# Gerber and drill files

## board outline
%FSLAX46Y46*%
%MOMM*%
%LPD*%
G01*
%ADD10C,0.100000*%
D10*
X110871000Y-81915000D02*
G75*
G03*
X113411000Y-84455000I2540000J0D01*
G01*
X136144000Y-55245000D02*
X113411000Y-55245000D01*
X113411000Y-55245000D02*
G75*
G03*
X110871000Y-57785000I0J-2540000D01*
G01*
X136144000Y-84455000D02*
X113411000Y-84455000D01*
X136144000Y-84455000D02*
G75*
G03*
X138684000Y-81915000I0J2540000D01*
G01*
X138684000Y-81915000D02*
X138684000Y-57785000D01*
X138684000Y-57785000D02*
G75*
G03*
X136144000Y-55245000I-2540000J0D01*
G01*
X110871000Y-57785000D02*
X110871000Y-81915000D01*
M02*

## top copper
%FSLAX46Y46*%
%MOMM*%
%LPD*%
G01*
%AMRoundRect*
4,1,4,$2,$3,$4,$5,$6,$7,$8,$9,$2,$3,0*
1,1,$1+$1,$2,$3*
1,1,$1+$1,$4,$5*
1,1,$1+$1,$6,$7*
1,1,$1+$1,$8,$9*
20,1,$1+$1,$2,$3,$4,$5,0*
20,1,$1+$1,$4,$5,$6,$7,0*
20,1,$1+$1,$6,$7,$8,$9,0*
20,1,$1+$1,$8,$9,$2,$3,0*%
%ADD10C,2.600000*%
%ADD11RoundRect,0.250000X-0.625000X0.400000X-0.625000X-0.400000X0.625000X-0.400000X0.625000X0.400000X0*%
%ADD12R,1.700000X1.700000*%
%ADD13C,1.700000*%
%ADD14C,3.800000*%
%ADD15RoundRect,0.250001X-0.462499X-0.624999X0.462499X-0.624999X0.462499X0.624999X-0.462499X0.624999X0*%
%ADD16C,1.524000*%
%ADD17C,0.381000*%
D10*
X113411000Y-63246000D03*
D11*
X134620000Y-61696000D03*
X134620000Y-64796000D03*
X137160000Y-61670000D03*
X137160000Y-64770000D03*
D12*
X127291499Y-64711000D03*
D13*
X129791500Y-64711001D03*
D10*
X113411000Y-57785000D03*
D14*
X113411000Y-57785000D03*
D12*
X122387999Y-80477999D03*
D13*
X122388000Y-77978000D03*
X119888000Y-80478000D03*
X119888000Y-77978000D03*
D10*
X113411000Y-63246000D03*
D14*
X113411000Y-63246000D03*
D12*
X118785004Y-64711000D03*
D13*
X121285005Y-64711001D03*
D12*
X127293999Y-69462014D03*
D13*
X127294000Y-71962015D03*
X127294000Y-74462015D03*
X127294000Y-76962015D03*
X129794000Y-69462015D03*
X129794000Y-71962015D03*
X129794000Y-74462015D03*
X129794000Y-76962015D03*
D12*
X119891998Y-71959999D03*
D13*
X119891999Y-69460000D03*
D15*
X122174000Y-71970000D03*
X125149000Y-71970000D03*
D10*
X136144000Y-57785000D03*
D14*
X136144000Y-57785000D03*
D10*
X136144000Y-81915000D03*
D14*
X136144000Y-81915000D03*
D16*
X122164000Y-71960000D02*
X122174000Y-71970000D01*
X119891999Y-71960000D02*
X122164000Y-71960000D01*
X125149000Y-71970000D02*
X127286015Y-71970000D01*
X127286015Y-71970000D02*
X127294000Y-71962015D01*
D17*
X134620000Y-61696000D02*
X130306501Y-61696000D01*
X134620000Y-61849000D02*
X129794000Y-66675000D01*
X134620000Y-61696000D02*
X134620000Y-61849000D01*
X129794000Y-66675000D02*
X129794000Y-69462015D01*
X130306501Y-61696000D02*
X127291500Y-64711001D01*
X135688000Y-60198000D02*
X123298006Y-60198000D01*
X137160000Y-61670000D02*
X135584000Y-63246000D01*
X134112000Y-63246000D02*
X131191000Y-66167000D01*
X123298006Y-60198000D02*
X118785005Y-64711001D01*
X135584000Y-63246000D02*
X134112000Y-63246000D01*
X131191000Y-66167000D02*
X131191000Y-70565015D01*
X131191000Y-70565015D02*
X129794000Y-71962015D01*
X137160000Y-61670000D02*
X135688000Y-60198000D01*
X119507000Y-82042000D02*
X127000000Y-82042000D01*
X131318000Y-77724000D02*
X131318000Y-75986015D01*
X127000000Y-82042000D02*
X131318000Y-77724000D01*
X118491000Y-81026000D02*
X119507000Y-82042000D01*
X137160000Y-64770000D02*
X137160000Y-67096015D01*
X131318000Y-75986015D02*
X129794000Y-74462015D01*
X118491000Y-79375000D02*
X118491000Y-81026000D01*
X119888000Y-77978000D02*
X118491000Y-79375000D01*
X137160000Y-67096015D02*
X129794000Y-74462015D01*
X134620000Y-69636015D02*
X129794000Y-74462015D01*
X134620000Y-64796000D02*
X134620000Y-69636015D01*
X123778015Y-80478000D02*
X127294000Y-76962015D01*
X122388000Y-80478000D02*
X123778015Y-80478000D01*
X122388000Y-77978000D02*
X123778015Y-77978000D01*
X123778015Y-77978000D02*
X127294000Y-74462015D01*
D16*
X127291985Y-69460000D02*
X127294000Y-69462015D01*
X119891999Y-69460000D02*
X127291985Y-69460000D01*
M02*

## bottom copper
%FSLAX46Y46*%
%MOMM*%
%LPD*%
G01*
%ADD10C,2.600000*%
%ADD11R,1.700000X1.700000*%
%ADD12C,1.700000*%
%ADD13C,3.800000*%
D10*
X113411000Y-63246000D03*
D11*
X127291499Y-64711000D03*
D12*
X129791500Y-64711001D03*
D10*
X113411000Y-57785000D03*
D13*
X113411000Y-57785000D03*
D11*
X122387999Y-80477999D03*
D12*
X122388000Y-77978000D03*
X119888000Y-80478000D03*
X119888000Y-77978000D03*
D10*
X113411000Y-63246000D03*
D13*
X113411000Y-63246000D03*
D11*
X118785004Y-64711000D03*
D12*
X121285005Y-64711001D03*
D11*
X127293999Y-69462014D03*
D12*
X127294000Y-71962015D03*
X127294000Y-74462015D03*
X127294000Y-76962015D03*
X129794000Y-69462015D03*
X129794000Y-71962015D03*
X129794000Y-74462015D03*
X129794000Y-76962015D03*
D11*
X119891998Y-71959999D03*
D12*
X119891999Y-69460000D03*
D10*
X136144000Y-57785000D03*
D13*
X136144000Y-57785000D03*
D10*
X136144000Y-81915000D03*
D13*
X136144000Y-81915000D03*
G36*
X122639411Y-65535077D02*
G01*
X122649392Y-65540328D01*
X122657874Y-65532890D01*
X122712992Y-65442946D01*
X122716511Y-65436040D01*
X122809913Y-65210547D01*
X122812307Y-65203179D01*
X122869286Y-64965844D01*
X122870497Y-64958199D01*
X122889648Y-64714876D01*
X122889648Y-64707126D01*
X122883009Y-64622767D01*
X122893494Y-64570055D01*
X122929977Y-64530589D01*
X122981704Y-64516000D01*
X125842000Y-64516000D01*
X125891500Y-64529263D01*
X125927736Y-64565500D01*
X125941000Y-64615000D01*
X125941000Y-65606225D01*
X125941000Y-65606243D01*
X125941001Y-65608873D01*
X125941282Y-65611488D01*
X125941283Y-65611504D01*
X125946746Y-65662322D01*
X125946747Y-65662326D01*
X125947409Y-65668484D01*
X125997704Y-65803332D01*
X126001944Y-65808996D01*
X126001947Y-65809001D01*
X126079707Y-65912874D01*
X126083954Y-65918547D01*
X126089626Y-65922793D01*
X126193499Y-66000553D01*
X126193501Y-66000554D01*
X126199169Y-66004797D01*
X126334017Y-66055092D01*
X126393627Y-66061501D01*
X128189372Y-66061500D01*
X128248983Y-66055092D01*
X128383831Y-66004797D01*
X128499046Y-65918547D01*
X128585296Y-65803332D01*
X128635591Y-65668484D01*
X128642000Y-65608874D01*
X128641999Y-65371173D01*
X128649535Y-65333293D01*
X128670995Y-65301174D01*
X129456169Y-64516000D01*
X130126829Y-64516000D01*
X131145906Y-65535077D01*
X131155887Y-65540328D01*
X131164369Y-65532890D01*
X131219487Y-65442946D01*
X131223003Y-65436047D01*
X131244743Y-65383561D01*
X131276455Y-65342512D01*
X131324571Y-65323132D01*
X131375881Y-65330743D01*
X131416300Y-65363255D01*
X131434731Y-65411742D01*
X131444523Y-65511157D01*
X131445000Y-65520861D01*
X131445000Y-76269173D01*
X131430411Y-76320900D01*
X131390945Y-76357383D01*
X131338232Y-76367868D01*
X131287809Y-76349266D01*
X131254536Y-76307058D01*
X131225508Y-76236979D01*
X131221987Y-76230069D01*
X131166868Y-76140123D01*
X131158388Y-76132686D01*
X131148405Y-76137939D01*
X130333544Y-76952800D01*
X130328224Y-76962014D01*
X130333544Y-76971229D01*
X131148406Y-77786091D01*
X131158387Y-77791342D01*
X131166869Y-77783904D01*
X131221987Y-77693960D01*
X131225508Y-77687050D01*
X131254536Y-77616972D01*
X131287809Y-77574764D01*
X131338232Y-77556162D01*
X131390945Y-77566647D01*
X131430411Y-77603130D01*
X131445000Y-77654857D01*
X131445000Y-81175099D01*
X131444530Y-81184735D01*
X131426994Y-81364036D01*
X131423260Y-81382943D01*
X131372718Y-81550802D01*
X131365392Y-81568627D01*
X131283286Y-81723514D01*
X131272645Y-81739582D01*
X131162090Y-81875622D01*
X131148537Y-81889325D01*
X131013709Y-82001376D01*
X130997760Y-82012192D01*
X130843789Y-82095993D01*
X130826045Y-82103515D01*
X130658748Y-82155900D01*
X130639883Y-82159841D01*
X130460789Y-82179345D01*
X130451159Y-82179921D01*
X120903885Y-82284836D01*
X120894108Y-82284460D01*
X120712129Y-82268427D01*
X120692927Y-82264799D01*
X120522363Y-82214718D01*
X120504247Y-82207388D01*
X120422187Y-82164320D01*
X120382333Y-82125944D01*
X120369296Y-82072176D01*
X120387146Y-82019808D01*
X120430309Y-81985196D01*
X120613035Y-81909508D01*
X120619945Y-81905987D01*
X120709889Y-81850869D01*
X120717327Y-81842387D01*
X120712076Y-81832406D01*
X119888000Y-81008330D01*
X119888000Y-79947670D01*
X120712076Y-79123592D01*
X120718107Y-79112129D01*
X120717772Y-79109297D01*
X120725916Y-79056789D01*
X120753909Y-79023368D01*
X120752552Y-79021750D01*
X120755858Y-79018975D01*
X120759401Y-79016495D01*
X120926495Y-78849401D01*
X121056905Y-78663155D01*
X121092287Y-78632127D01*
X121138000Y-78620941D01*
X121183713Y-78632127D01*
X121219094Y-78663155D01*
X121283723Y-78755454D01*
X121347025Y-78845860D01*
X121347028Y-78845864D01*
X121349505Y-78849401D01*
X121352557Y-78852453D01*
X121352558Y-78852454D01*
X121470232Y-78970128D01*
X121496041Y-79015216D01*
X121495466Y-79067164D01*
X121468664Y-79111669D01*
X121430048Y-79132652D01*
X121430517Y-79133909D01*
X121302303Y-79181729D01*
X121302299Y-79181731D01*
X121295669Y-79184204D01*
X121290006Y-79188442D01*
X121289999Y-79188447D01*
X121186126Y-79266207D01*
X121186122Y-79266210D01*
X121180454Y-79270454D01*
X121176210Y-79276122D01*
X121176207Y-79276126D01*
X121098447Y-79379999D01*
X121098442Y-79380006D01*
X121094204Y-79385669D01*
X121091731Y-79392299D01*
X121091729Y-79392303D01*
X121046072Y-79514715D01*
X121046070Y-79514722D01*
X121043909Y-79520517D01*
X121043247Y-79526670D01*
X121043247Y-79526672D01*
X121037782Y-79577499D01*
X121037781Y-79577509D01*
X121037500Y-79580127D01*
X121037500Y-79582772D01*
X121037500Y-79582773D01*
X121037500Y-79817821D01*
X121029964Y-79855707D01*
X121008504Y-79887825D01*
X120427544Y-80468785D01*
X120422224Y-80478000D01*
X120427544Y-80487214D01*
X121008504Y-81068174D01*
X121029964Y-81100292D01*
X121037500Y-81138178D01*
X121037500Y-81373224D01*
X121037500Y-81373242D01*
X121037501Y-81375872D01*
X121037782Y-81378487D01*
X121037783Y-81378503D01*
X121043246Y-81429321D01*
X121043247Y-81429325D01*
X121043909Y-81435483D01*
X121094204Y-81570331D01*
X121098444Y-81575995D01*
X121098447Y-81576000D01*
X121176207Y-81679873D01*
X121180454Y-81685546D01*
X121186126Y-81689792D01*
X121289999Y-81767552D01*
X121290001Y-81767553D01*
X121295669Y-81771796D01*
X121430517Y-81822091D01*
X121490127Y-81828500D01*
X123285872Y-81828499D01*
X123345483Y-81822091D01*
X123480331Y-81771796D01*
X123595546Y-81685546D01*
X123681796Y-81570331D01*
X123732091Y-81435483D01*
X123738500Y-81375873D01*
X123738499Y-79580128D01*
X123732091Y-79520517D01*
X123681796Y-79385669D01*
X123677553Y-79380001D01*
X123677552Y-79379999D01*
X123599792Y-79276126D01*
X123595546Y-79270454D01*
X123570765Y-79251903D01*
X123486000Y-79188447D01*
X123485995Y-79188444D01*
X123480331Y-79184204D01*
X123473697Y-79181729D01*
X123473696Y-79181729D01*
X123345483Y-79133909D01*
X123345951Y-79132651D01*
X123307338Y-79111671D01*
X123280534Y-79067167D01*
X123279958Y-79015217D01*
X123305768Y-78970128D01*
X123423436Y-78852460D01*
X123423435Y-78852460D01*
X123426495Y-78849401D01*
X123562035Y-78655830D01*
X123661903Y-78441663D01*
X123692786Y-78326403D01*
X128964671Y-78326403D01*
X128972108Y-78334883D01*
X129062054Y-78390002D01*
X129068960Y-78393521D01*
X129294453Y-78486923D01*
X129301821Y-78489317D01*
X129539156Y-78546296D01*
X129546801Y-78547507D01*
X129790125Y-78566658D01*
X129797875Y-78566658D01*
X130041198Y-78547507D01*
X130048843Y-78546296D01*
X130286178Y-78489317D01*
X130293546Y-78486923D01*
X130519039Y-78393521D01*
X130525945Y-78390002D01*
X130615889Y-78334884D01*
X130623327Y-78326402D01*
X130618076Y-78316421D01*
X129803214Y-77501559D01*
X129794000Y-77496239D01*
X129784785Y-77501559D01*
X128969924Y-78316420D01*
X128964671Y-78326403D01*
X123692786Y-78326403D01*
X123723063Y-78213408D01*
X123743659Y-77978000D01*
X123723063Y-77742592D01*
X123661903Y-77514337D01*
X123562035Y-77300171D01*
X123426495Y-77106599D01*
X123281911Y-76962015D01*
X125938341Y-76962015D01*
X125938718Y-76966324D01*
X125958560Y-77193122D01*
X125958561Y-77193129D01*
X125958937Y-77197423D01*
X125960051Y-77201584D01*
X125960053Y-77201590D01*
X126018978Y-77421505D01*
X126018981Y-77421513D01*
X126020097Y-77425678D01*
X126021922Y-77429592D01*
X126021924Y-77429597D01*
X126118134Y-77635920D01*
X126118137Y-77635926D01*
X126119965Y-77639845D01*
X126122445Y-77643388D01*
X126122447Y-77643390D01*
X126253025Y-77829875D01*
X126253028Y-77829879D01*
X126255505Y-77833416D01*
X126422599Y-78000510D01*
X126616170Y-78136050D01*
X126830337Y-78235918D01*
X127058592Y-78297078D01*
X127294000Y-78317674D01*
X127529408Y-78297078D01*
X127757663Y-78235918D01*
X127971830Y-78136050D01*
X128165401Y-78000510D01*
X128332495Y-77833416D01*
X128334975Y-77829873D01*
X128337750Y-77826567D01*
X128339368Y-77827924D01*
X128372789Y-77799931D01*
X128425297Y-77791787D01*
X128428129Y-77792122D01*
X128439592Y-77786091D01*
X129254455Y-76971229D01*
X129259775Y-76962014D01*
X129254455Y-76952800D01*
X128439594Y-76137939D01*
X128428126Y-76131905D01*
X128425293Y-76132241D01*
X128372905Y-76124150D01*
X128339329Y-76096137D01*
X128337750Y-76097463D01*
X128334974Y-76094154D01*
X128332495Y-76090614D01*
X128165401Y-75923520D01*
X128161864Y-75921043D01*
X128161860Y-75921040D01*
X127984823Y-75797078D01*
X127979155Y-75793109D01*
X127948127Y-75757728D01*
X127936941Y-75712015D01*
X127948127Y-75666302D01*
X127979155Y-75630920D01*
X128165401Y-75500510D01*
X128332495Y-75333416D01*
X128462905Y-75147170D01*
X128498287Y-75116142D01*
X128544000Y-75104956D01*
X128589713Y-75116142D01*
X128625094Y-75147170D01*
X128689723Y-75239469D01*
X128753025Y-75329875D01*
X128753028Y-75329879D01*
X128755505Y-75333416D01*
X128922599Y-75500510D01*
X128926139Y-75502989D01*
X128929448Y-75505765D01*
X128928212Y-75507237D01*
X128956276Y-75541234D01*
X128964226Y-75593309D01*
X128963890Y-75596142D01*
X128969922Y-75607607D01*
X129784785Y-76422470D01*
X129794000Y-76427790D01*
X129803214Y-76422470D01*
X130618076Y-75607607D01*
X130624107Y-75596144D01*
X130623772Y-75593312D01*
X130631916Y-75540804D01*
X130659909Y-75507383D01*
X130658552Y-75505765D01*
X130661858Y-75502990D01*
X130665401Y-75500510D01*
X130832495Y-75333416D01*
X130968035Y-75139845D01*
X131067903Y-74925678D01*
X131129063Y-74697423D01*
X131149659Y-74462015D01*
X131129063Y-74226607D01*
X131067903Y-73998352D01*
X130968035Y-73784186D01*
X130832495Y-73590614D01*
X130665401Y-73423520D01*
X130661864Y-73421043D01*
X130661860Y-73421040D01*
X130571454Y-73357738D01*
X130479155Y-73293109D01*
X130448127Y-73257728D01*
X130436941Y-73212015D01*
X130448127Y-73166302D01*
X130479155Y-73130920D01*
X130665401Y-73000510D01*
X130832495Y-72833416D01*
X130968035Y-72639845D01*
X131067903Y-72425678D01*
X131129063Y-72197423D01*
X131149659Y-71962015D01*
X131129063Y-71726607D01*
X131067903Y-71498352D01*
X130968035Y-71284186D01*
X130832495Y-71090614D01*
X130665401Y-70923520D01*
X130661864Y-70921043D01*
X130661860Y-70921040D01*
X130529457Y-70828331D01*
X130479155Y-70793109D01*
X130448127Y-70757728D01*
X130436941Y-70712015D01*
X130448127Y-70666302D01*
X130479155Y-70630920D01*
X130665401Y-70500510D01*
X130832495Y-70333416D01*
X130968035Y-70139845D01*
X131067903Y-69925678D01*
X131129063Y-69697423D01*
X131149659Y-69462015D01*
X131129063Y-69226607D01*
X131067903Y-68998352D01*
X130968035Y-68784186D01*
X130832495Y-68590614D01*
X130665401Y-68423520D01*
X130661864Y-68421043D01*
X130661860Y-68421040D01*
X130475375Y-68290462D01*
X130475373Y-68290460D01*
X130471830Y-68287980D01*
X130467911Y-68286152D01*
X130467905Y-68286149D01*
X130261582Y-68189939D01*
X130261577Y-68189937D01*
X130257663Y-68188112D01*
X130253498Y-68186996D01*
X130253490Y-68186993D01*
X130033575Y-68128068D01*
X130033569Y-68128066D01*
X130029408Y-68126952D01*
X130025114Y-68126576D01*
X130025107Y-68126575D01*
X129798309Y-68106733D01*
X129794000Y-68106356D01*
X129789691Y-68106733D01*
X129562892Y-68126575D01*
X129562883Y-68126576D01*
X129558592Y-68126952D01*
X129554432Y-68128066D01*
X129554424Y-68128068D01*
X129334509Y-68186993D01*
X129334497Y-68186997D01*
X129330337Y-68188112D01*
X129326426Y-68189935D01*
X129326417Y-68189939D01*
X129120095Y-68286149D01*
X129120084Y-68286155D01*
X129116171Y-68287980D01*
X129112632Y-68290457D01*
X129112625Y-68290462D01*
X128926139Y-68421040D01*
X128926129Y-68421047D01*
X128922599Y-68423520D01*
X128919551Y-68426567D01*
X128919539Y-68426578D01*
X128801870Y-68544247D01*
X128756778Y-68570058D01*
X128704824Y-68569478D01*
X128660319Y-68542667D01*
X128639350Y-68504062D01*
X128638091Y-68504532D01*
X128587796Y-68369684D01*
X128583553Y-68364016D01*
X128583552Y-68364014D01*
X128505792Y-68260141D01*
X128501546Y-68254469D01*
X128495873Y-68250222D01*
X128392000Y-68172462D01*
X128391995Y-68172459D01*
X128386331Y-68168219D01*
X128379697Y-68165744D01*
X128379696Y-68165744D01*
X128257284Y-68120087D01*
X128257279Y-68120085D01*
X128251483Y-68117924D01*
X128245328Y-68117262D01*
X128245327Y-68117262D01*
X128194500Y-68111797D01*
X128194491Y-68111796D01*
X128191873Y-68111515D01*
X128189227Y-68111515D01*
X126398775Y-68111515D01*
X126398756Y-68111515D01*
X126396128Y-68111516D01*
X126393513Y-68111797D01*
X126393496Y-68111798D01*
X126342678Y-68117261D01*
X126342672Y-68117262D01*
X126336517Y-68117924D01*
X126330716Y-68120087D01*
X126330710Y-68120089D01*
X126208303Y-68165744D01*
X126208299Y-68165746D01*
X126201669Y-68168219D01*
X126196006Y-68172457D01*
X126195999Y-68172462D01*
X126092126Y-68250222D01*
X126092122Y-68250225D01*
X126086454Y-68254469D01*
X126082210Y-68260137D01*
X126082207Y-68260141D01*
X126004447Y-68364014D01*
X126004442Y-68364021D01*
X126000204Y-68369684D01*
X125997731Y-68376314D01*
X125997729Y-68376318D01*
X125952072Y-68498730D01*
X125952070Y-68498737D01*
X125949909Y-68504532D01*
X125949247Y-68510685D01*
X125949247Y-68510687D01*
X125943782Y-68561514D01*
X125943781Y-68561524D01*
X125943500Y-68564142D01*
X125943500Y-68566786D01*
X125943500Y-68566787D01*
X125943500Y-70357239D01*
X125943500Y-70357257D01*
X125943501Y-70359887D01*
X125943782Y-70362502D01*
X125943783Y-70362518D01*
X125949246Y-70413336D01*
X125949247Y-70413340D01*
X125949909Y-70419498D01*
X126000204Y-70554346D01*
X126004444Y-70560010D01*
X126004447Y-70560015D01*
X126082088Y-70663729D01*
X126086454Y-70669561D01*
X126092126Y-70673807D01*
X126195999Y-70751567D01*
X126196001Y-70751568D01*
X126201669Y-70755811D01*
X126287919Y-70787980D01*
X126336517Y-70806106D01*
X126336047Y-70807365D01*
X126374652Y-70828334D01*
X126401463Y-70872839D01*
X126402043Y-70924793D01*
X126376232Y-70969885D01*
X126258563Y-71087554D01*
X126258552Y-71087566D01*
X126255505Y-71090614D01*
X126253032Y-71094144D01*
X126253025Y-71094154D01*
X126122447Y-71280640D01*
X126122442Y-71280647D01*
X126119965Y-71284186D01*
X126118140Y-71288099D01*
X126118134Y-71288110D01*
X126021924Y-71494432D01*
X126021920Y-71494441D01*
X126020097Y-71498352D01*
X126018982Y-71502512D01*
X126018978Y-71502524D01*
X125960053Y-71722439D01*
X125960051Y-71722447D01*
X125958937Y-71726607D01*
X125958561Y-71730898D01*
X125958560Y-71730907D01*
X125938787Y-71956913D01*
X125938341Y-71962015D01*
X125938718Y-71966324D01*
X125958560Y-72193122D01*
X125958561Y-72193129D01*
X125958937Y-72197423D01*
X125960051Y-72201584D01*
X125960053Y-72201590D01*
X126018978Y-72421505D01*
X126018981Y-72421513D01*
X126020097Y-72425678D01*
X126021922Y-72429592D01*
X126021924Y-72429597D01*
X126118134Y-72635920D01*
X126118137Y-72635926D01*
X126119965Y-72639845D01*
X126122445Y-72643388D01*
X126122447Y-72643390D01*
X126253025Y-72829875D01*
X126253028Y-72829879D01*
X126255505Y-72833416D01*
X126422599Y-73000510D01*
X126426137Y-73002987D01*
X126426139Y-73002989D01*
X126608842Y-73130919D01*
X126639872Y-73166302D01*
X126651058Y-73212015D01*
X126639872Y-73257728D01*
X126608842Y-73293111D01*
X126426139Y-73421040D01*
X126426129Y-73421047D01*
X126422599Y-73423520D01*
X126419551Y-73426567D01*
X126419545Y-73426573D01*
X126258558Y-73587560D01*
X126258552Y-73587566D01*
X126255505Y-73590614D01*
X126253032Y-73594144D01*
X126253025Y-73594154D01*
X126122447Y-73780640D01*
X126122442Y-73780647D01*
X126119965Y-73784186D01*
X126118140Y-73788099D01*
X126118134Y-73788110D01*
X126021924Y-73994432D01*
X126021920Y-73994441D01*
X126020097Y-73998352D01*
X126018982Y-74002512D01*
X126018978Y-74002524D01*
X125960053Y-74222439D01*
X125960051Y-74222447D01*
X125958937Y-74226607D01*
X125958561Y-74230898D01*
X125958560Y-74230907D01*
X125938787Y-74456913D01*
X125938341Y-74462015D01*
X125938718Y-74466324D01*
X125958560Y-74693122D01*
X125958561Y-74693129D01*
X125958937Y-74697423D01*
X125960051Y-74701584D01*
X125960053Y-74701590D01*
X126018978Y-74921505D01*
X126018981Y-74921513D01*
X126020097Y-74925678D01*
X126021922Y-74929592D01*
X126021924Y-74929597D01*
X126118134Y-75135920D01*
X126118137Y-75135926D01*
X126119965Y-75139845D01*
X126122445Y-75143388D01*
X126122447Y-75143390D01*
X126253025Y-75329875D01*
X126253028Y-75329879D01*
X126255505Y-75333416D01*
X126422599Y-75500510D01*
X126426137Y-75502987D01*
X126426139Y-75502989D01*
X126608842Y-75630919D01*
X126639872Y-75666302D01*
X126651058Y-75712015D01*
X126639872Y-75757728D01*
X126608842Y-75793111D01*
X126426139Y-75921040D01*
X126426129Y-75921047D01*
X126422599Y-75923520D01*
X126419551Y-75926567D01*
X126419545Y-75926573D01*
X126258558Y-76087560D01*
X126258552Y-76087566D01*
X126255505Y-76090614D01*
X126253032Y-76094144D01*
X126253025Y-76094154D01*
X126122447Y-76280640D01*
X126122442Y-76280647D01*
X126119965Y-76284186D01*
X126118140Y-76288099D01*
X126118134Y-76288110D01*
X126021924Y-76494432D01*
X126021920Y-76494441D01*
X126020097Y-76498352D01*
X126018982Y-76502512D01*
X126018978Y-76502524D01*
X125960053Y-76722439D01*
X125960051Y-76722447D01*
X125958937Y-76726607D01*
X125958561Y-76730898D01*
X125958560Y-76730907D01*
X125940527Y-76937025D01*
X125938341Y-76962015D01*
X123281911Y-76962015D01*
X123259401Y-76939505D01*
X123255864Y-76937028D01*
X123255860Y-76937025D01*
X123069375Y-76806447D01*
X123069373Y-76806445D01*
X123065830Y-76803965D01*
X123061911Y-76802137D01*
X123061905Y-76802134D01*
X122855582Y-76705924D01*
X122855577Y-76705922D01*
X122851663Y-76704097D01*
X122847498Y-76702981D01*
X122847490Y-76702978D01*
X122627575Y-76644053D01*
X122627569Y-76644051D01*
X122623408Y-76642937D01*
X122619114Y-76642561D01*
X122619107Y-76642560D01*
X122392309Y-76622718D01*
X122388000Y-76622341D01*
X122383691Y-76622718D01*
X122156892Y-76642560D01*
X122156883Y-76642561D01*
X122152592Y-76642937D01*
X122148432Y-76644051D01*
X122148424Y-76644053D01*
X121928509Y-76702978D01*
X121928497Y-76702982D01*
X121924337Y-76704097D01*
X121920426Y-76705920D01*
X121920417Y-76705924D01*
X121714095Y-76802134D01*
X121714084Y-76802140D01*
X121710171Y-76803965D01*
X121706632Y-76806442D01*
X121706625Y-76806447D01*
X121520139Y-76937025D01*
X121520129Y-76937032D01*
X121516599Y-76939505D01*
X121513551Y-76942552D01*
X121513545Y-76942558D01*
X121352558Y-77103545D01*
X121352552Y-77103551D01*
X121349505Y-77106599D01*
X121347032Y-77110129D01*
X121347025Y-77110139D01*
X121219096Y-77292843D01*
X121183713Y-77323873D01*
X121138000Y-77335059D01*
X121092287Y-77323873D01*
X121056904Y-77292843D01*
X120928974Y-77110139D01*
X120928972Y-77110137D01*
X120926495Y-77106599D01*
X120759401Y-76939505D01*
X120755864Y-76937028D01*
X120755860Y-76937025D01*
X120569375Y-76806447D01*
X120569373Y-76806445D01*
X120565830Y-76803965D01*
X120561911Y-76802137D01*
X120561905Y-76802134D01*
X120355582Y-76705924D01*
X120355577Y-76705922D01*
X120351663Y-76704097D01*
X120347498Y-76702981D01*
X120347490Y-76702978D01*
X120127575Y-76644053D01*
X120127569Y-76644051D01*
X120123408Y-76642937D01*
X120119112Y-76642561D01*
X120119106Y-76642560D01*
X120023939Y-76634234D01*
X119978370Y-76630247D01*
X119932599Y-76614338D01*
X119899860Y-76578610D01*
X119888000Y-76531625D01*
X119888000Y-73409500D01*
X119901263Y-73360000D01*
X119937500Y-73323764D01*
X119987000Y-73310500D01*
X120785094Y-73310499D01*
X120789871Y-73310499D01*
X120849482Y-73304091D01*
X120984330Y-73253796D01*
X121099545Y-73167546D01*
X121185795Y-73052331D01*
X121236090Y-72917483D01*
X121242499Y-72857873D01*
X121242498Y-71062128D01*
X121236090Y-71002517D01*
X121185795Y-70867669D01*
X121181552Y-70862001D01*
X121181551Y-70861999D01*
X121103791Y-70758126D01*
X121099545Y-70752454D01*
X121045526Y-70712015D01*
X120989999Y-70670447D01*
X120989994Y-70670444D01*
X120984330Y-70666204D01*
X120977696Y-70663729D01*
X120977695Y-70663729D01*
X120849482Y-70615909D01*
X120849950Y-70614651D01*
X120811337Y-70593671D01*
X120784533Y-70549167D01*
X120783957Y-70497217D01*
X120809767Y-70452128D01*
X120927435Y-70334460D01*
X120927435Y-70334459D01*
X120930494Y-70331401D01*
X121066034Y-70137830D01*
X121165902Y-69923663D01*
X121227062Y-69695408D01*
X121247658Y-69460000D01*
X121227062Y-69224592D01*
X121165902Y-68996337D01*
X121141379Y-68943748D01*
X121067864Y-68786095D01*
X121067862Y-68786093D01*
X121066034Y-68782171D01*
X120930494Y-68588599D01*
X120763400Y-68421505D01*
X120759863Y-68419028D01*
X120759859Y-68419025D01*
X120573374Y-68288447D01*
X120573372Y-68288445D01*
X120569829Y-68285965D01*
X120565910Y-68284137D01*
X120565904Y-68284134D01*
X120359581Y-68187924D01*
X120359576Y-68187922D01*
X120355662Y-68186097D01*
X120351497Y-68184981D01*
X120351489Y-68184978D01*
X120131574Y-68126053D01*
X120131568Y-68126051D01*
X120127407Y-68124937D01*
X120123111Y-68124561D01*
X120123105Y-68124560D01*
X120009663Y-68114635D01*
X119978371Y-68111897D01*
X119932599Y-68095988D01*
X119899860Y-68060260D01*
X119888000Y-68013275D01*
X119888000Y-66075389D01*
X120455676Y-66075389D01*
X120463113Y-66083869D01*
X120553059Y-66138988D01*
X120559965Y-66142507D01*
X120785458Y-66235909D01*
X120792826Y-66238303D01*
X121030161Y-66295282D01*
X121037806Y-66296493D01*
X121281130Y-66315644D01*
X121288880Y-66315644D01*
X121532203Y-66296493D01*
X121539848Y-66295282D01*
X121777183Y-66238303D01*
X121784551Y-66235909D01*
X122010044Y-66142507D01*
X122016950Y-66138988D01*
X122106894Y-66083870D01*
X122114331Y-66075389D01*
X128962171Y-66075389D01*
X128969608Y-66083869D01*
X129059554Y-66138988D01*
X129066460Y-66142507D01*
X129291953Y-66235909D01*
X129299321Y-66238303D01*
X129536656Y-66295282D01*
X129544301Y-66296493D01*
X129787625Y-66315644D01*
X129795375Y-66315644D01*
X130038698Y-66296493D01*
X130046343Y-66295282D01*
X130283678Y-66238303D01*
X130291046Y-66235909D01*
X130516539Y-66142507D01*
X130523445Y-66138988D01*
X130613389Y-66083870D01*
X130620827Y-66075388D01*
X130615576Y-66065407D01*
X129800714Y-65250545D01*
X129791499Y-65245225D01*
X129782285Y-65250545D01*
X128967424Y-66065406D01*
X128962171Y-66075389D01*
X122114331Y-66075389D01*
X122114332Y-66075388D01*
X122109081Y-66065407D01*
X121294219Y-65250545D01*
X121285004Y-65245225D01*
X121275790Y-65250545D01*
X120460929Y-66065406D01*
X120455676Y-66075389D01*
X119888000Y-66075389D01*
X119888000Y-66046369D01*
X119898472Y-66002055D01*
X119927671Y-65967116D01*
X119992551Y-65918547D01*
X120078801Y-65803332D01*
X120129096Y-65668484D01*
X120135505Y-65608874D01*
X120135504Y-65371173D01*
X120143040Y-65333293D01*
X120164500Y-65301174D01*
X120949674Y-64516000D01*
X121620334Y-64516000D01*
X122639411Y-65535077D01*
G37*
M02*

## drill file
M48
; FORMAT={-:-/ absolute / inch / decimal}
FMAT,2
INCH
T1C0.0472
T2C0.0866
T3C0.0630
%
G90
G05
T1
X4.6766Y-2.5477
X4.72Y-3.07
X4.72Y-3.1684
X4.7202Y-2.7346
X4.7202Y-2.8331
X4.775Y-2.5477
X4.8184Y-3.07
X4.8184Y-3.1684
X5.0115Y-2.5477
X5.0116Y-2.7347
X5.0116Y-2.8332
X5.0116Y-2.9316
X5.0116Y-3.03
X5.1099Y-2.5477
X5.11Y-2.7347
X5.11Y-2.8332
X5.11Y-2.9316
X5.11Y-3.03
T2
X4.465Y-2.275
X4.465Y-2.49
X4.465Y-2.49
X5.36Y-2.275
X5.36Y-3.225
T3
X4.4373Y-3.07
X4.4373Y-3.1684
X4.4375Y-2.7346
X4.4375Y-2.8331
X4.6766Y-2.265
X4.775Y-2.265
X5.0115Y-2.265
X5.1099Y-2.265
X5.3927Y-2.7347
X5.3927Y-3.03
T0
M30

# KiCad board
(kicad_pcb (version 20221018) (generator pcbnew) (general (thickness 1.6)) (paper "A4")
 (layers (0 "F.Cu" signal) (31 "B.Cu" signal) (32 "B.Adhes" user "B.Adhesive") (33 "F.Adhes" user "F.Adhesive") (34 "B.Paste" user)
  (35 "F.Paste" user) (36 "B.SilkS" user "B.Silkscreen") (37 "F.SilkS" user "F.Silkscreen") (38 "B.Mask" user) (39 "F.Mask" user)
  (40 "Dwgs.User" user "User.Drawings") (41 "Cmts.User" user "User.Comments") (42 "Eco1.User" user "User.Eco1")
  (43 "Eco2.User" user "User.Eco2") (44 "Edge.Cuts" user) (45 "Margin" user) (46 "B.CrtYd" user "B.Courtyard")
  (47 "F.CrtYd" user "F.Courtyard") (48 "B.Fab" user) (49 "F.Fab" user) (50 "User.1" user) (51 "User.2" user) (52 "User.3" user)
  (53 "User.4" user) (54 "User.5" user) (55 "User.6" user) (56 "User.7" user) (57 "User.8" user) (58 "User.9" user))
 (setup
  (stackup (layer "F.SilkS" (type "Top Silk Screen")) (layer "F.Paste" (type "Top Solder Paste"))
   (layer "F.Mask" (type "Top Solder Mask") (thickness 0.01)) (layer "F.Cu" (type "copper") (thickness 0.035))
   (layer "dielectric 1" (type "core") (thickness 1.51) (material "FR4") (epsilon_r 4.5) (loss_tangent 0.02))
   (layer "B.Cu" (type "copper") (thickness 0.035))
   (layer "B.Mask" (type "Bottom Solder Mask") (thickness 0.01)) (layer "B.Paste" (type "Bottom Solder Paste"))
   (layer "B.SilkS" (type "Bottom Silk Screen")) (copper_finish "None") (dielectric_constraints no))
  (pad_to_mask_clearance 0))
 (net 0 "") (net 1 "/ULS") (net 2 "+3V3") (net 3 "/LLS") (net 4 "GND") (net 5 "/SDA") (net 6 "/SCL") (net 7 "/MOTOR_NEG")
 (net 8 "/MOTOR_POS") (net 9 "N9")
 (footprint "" (layer "F.Cu") (at 113.411 63.246)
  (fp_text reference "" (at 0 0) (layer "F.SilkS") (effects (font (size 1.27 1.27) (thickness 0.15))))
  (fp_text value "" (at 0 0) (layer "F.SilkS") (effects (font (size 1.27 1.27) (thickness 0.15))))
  (pad "1" thru_hole circle (at 0 0) (size 2.6 2.6) (drill 2.2) (layers "*.Cu" "*.Mask")))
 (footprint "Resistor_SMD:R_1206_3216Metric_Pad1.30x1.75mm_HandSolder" (layer "F.Cu") (at 134.62 63.246 -90)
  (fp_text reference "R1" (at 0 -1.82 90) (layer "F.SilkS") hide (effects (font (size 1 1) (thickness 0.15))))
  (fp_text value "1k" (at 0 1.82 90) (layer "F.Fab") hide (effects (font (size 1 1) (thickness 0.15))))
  (pad "1" smd roundrect (at -1.55 0 270) (size 1.3 1.75) (layers "F.Cu" "F.Paste" "F.Mask") (roundrect_rratio 0.1923076923) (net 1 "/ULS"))
  (pad "2" smd roundrect (at 1.55 0 270) (size 1.3 1.75) (layers "F.Cu" "F.Paste" "F.Mask") (roundrect_rratio 0.1923076923) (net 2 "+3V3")))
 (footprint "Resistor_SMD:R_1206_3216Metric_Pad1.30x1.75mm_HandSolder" (layer "F.Cu") (at 137.16 63.22 -90)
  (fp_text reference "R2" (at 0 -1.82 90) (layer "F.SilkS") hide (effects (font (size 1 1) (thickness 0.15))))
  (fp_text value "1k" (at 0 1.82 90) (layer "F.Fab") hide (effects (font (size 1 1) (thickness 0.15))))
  (pad "1" smd roundrect (at -1.55 0 270) (size 1.3 1.75) (layers "F.Cu" "F.Paste" "F.Mask") (roundrect_rratio 0.1923076923) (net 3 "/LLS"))
  (pad "2" smd roundrect (at 1.55 0 270) (size 1.3 1.75) (layers "F.Cu" "F.Paste" "F.Mask") (roundrect_rratio 0.1923076923) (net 2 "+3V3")))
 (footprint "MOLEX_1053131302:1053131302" (layer "F.Cu") (at 127.2915 64.711001 180)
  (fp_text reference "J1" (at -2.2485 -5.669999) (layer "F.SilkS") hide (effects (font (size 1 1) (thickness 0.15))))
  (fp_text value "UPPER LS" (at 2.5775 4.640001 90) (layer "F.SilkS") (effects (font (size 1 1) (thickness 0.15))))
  (pad "" np_thru_hole circle (at -2.499995 7.180001 180) (size 1.6 1.6) (drill 1.6) (layers "*.Cu" "*.Mask"))
  (pad "" np_thru_hole circle (at 0 7.180001 180) (size 1.6 1.6) (drill 1.6) (layers "*.Cu" "*.Mask"))
  (pad "1" thru_hole rect (at 0 0 180) (size 1.7 1.7) (drill 1.2) (layers "*.Cu" "*.Mask") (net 1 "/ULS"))
  (pad "2" thru_hole circle (at -2.5 0 180) (size 1.7 1.7) (drill 1.2) (layers "*.Cu" "*.Mask") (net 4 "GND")))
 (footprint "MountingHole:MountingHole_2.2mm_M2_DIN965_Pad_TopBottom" (layer "F.Cu") (at 113.411 57.785)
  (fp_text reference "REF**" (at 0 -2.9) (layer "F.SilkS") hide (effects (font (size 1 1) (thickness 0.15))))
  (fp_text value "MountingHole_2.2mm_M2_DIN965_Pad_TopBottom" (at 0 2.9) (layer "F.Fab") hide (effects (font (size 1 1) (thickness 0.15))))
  (pad "1" thru_hole circle (at 0 0) (size 2.6 2.6) (drill 2.2) (layers "*.Cu" "*.Mask"))
  (pad "1" connect circle (at 0 0) (size 3.8 3.8) (layers "F.Cu" "F.Mask"))
  (pad "1" connect circle (at 0 0) (size 3.8 3.8) (layers "B.Cu" "B.Mask")))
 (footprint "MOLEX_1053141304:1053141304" (layer "F.Cu") (at 122.388 80.478 -90)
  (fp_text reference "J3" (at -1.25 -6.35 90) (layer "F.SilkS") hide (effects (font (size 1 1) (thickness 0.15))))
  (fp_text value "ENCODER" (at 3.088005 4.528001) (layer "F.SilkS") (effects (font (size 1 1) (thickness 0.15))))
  (pad "" np_thru_hole circle (at -2.499995 9.680001 270) (size 1.6 1.6) (drill 1.6) (layers "*.Cu" "*.Mask"))
  (pad "" np_thru_hole circle (at 0 9.680001 270) (size 1.6 1.6) (drill 1.6) (layers "*.Cu" "*.Mask"))
  (pad "1" thru_hole rect (at 0 0 270) (size 1.7 1.7) (drill 1.2) (layers "*.Cu" "*.Mask") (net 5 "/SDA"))
  (pad "2" thru_hole circle (at -2.5 0 270) (size 1.7 1.7) (drill 1.2) (layers "*.Cu" "*.Mask") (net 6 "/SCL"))
  (pad "3" thru_hole circle (at 0 2.5 270) (size 1.7 1.7) (drill 1.2) (layers "*.Cu" "*.Mask") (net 4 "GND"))
  (pad "4" thru_hole circle (at -2.5 2.5 270) (size 1.7 1.7) (drill 1.2) (layers "*.Cu" "*.Mask") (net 2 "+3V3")))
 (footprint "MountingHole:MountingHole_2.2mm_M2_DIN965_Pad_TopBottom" (layer "F.Cu") (at 113.411 63.246)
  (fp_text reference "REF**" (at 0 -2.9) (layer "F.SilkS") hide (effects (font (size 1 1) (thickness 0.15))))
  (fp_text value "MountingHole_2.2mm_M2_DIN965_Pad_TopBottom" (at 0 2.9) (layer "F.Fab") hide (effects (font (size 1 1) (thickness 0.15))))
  (pad "1" thru_hole circle (at 0 0) (size 2.6 2.6) (drill 2.2) (layers "*.Cu" "*.Mask"))
  (pad "1" connect circle (at 0 0) (size 3.8 3.8) (layers "F.Cu" "F.Mask"))
  (pad "1" connect circle (at 0 0) (size 3.8 3.8) (layers "B.Cu" "B.Mask")))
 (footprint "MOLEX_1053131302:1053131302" (layer "F.Cu") (at 118.785005 64.711001 180)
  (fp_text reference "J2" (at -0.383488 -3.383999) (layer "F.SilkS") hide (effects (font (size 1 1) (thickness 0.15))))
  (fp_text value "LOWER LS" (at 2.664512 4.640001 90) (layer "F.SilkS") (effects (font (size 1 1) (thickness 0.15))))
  (pad "" np_thru_hole circle (at -2.499995 7.180001 180) (size 1.6 1.6) (drill 1.6) (layers "*.Cu" "*.Mask"))
  (pad "" np_thru_hole circle (at 0 7.180001 180) (size 1.6 1.6) (drill 1.6) (layers "*.Cu" "*.Mask"))
  (pad "1" thru_hole rect (at 0 0 180) (size 1.7 1.7) (drill 1.2) (layers "*.Cu" "*.Mask") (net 3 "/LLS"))
  (pad "2" thru_hole circle (at -2.5 0 180) (size 1.7 1.7) (drill 1.2) (layers "*.Cu" "*.Mask") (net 4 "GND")))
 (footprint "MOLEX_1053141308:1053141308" (layer "F.Cu") (at 127.294 69.462015 90)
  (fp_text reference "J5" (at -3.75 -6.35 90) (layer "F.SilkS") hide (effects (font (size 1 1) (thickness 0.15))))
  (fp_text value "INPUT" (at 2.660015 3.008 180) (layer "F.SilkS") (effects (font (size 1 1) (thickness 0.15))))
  (pad "" np_thru_hole circle (at -7.499985 9.680001 90) (size 1.6 1.6) (drill 1.6) (layers "*.Cu" "*.Mask"))
  (pad "" np_thru_hole circle (at 0 9.680001 90) (size 1.6 1.6) (drill 1.6) (layers "*.Cu" "*.Mask"))
  (pad "1" thru_hole rect (at 0 0 90) (size 1.7 1.7) (drill 1.2) (layers "*.Cu" "*.Mask") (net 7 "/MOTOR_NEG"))
  (pad "2" thru_hole circle (at -2.5 0 90) (size 1.7 1.7) (drill 1.2) (layers "*.Cu" "*.Mask") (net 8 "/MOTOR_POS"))
  (pad "3" thru_hole circle (at -5 0 90) (size 1.7 1.7) (drill 1.2) (layers "*.Cu" "*.Mask") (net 6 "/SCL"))
  (pad "4" thru_hole circle (at -7.5 0 90) (size 1.7 1.7) (drill 1.2) (layers "*.Cu" "*.Mask") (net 5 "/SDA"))
  (pad "5" thru_hole circle (at 0 2.5 90) (size 1.7 1.7) (drill 1.2) (layers "*.Cu" "*.Mask") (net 1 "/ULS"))
  (pad "6" thru_hole circle (at -2.5 2.5 90) (size 1.7 1.7) (drill 1.2) (layers "*.Cu" "*.Mask") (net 3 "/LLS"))
  (pad "7" thru_hole circle (at -5 2.5 90) (size 1.7 1.7) (drill 1.2) (layers "*.Cu" "*.Mask") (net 2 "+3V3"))
  (pad "8" thru_hole circle (at -7.5 2.5 90) (size 1.7 1.7) (drill 1.2) (layers "*.Cu" "*.Mask") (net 4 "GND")))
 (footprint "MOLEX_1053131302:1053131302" (layer "F.Cu") (at 119.891999 71.96 -90)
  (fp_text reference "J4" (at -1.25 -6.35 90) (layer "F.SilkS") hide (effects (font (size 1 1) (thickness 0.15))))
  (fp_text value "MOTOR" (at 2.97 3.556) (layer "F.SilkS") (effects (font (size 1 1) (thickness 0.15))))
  (pad "" np_thru_hole circle (at -2.499995 7.180001 270) (size 1.6 1.6) (drill 1.6) (layers "*.Cu" "*.Mask"))
  (pad "" np_thru_hole circle (at 0 7.180001 270) (size 1.6 1.6) (drill 1.6) (layers "*.Cu" "*.Mask"))
  (pad "1" thru_hole rect (at 0 0 270) (size 1.7 1.7) (drill 1.2) (layers "*.Cu" "*.Mask") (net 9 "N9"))
  (pad "2" thru_hole circle (at -2.5 0 270) (size 1.7 1.7) (drill 1.2) (layers "*.Cu" "*.Mask") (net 7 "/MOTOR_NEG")))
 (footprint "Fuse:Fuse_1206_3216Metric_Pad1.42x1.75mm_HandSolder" (layer "F.Cu") (at 123.6615 71.97)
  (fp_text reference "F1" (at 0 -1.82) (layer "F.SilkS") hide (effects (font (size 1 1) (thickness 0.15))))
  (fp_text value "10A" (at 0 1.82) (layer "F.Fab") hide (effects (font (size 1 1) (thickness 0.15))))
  (pad "1" smd roundrect (at -1.4875 0) (size 1.425 1.75) (layers "F.Cu" "F.Paste" "F.Mask") (roundrect_rratio 0.1754392982) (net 9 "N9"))
  (pad "2" smd roundrect (at 1.4875 0) (size 1.425 1.75) (layers "F.Cu" "F.Paste" "F.Mask") (roundrect_rratio 0.1754392982)
   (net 8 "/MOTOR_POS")))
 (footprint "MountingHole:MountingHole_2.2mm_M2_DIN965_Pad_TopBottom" (layer "F.Cu") (at 136.144 57.785)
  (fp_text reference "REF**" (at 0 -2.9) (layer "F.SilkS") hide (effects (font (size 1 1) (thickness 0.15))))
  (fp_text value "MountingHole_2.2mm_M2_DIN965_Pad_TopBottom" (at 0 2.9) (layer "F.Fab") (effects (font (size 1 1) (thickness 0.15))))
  (pad "1" thru_hole circle (at 0 0) (size 2.6 2.6) (drill 2.2) (layers "*.Cu" "*.Mask"))
  (pad "1" connect circle (at 0 0) (size 3.8 3.8) (layers "F.Cu" "F.Mask"))
  (pad "1" connect circle (at 0 0) (size 3.8 3.8) (layers "B.Cu" "B.Mask")))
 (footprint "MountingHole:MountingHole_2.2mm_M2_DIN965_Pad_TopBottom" (layer "F.Cu") (at 136.144 81.915)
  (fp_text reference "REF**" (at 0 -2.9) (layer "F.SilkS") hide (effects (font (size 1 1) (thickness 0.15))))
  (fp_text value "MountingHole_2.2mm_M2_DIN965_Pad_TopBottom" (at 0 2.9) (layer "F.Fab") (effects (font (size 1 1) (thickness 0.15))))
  (pad "1" thru_hole circle (at 0 0) (size 2.6 2.6) (drill 2.2) (layers "*.Cu" "*.Mask"))
  (pad "1" connect circle (at 0 0) (size 3.8 3.8) (layers "F.Cu" "F.Mask"))
  (pad "1" connect circle (at 0 0) (size 3.8 3.8) (layers "B.Cu" "B.Mask")))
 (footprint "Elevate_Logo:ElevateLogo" (layer "B.Cu") (at 124.841 58.42 180)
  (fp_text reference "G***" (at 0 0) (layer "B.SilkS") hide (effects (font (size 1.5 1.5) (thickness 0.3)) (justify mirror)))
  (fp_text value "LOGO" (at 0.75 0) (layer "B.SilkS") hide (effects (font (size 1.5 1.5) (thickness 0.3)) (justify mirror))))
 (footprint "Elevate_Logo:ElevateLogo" (layer "B.Cu") (at 124.841 75.565 180)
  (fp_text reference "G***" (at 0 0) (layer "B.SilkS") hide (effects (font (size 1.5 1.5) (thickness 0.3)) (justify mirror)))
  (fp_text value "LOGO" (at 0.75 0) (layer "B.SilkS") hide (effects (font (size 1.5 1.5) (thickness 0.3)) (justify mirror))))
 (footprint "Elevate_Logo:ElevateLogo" (layer "B.Cu") (at 124.841 69.85 180)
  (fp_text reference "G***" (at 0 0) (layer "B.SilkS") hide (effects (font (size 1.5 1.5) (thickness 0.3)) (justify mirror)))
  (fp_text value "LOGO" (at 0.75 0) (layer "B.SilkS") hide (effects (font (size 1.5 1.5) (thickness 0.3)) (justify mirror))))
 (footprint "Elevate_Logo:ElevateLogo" (layer "B.Cu") (at 124.841 64.135 180)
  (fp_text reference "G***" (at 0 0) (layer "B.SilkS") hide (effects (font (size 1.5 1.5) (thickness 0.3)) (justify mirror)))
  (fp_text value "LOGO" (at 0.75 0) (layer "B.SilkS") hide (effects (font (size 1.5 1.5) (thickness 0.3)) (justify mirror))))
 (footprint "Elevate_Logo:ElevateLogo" (layer "B.Cu") (at 124.841 81.28 180)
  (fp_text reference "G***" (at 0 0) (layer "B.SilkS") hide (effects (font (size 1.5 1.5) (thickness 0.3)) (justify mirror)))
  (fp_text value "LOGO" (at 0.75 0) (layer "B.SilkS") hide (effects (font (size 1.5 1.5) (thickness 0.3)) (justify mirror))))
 (gr_arc (start 113.411 84.455) (mid 111.614949 83.711051) (end 110.871 81.915) (stroke (width 0.1) (type default)) (layer "Edge.Cuts"))
 (gr_line (start 136.144 55.245) (end 113.411 55.245) (stroke (width 0.1) (type default)) (layer "Edge.Cuts"))
 (gr_arc (start 110.871 57.785) (mid 111.614949 55.988949) (end 113.411 55.245) (stroke (width 0.1) (type default)) (layer "Edge.Cuts"))
 (gr_line (start 136.144 84.455) (end 113.411 84.455) (stroke (width 0.1) (type default)) (layer "Edge.Cuts"))
 (gr_arc (start 138.684 81.915) (mid 137.940051 83.711051) (end 136.144 84.455) (stroke (width 0.1) (type default)) (layer "Edge.Cuts"))
 (gr_line (start 138.684 81.915) (end 138.684 57.785) (stroke (width 0.1) (type default)) (layer "Edge.Cuts"))
 (gr_arc (start 136.144 55.245) (mid 137.940051 55.988949) (end 138.684 57.785) (stroke (width 0.1) (type default)) (layer "Edge.Cuts"))
 (gr_line (start 110.871 57.785) (end 110.871 81.915) (stroke (width 0.1) (type default)) (layer "Edge.Cuts"))
 (segment (start 122.164 71.96) (end 122.174 71.97) (width 1.524) (layer "F.Cu") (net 9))
 (segment (start 119.891999 71.96) (end 122.164 71.96) (width 1.524) (layer "F.Cu") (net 9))
 (segment (start 125.149 71.97) (end 127.286015 71.97) (width 1.524) (layer "F.Cu") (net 8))
 (segment (start 127.286015 71.97) (end 127.294 71.962015) (width 1.524) (layer "F.Cu") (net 8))
 (segment (start 134.62 61.696) (end 130.306501 61.696) (width 0.381) (layer "F.Cu") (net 1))
 (segment (start 134.62 61.849) (end 129.794 66.675) (width 0.381) (layer "F.Cu") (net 1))
 (segment (start 134.62 61.696) (end 134.62 61.849) (width 0.381) (layer "F.Cu") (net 1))
 (segment (start 129.794 66.675) (end 129.794 69.462015) (width 0.381) (layer "F.Cu") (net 1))
 (segment (start 130.306501 61.696) (end 127.2915 64.711001) (width 0.381) (layer "F.Cu") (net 1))
 (segment (start 135.688 60.198) (end 123.298006 60.198) (width 0.381) (layer "F.Cu") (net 3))
 (segment (start 137.16 61.67) (end 135.584 63.246) (width 0.381) (layer "F.Cu") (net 3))
 (segment (start 134.112 63.246) (end 131.191 66.167) (width 0.381) (layer "F.Cu") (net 3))
 (segment (start 123.298006 60.198) (end 118.785005 64.711001) (width 0.381) (layer "F.Cu") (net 3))
 (segment (start 135.584 63.246) (end 134.112 63.246) (width 0.381) (layer "F.Cu") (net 3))
 (segment (start 131.191 66.167) (end 131.191 70.565015) (width 0.381) (layer "F.Cu") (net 3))
 (segment (start 131.191 70.565015) (end 129.794 71.962015) (width 0.381) (layer "F.Cu") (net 3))
 (segment (start 137.16 61.67) (end 135.688 60.198) (width 0.381) (layer "F.Cu") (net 3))
 (segment (start 119.507 82.042) (end 127 82.042) (width 0.381) (layer "F.Cu") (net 2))
 (segment (start 131.318 77.724) (end 131.318 75.986015) (width 0.381) (layer "F.Cu") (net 2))
 (segment (start 127 82.042) (end 131.318 77.724) (width 0.381) (layer "F.Cu") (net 2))
 (segment (start 118.491 81.026) (end 119.507 82.042) (width 0.381) (layer "F.Cu") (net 2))
 (segment (start 137.16 64.77) (end 137.16 67.096015) (width 0.381) (layer "F.Cu") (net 2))
 (segment (start 131.318 75.986015) (end 129.794 74.462015) (width 0.381) (layer "F.Cu") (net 2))
 (segment (start 118.491 79.375) (end 118.491 81.026) (width 0.381) (layer "F.Cu") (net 2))
 (segment (start 119.888 77.978) (end 118.491 79.375) (width 0.381) (layer "F.Cu") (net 2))
 (segment (start 137.16 67.096015) (end 129.794 74.462015) (width 0.381) (layer "F.Cu") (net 2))
 (segment (start 134.62 69.636015) (end 129.794 74.462015) (width 0.381) (layer "F.Cu") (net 2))
 (segment (start 134.62 64.796) (end 134.62 69.636015) (width 0.381) (layer "F.Cu") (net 2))
 (segment (start 123.778015 80.478) (end 127.294 76.962015) (width 0.381) (layer "F.Cu") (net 5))
 (segment (start 122.388 80.478) (end 123.778015 80.478) (width 0.381) (layer "F.Cu") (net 5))
 (segment (start 122.388 77.978) (end 123.778015 77.978) (width 0.381) (layer "F.Cu") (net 6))
 (segment (start 123.778015 77.978) (end 127.294 74.462015) (width 0.381) (layer "F.Cu") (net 6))
 (segment (start 127.291985 69.46) (end 127.294 69.462015) (width 1.524) (layer "F.Cu") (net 7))
 (segment (start 119.891999 69.46) (end 127.291985 69.46) (width 1.524) (layer "F.Cu") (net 7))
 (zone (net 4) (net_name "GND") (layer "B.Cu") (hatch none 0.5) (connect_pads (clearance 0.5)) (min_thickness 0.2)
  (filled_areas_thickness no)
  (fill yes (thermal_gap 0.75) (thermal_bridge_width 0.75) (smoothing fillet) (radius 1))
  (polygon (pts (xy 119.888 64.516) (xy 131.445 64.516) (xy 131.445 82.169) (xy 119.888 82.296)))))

